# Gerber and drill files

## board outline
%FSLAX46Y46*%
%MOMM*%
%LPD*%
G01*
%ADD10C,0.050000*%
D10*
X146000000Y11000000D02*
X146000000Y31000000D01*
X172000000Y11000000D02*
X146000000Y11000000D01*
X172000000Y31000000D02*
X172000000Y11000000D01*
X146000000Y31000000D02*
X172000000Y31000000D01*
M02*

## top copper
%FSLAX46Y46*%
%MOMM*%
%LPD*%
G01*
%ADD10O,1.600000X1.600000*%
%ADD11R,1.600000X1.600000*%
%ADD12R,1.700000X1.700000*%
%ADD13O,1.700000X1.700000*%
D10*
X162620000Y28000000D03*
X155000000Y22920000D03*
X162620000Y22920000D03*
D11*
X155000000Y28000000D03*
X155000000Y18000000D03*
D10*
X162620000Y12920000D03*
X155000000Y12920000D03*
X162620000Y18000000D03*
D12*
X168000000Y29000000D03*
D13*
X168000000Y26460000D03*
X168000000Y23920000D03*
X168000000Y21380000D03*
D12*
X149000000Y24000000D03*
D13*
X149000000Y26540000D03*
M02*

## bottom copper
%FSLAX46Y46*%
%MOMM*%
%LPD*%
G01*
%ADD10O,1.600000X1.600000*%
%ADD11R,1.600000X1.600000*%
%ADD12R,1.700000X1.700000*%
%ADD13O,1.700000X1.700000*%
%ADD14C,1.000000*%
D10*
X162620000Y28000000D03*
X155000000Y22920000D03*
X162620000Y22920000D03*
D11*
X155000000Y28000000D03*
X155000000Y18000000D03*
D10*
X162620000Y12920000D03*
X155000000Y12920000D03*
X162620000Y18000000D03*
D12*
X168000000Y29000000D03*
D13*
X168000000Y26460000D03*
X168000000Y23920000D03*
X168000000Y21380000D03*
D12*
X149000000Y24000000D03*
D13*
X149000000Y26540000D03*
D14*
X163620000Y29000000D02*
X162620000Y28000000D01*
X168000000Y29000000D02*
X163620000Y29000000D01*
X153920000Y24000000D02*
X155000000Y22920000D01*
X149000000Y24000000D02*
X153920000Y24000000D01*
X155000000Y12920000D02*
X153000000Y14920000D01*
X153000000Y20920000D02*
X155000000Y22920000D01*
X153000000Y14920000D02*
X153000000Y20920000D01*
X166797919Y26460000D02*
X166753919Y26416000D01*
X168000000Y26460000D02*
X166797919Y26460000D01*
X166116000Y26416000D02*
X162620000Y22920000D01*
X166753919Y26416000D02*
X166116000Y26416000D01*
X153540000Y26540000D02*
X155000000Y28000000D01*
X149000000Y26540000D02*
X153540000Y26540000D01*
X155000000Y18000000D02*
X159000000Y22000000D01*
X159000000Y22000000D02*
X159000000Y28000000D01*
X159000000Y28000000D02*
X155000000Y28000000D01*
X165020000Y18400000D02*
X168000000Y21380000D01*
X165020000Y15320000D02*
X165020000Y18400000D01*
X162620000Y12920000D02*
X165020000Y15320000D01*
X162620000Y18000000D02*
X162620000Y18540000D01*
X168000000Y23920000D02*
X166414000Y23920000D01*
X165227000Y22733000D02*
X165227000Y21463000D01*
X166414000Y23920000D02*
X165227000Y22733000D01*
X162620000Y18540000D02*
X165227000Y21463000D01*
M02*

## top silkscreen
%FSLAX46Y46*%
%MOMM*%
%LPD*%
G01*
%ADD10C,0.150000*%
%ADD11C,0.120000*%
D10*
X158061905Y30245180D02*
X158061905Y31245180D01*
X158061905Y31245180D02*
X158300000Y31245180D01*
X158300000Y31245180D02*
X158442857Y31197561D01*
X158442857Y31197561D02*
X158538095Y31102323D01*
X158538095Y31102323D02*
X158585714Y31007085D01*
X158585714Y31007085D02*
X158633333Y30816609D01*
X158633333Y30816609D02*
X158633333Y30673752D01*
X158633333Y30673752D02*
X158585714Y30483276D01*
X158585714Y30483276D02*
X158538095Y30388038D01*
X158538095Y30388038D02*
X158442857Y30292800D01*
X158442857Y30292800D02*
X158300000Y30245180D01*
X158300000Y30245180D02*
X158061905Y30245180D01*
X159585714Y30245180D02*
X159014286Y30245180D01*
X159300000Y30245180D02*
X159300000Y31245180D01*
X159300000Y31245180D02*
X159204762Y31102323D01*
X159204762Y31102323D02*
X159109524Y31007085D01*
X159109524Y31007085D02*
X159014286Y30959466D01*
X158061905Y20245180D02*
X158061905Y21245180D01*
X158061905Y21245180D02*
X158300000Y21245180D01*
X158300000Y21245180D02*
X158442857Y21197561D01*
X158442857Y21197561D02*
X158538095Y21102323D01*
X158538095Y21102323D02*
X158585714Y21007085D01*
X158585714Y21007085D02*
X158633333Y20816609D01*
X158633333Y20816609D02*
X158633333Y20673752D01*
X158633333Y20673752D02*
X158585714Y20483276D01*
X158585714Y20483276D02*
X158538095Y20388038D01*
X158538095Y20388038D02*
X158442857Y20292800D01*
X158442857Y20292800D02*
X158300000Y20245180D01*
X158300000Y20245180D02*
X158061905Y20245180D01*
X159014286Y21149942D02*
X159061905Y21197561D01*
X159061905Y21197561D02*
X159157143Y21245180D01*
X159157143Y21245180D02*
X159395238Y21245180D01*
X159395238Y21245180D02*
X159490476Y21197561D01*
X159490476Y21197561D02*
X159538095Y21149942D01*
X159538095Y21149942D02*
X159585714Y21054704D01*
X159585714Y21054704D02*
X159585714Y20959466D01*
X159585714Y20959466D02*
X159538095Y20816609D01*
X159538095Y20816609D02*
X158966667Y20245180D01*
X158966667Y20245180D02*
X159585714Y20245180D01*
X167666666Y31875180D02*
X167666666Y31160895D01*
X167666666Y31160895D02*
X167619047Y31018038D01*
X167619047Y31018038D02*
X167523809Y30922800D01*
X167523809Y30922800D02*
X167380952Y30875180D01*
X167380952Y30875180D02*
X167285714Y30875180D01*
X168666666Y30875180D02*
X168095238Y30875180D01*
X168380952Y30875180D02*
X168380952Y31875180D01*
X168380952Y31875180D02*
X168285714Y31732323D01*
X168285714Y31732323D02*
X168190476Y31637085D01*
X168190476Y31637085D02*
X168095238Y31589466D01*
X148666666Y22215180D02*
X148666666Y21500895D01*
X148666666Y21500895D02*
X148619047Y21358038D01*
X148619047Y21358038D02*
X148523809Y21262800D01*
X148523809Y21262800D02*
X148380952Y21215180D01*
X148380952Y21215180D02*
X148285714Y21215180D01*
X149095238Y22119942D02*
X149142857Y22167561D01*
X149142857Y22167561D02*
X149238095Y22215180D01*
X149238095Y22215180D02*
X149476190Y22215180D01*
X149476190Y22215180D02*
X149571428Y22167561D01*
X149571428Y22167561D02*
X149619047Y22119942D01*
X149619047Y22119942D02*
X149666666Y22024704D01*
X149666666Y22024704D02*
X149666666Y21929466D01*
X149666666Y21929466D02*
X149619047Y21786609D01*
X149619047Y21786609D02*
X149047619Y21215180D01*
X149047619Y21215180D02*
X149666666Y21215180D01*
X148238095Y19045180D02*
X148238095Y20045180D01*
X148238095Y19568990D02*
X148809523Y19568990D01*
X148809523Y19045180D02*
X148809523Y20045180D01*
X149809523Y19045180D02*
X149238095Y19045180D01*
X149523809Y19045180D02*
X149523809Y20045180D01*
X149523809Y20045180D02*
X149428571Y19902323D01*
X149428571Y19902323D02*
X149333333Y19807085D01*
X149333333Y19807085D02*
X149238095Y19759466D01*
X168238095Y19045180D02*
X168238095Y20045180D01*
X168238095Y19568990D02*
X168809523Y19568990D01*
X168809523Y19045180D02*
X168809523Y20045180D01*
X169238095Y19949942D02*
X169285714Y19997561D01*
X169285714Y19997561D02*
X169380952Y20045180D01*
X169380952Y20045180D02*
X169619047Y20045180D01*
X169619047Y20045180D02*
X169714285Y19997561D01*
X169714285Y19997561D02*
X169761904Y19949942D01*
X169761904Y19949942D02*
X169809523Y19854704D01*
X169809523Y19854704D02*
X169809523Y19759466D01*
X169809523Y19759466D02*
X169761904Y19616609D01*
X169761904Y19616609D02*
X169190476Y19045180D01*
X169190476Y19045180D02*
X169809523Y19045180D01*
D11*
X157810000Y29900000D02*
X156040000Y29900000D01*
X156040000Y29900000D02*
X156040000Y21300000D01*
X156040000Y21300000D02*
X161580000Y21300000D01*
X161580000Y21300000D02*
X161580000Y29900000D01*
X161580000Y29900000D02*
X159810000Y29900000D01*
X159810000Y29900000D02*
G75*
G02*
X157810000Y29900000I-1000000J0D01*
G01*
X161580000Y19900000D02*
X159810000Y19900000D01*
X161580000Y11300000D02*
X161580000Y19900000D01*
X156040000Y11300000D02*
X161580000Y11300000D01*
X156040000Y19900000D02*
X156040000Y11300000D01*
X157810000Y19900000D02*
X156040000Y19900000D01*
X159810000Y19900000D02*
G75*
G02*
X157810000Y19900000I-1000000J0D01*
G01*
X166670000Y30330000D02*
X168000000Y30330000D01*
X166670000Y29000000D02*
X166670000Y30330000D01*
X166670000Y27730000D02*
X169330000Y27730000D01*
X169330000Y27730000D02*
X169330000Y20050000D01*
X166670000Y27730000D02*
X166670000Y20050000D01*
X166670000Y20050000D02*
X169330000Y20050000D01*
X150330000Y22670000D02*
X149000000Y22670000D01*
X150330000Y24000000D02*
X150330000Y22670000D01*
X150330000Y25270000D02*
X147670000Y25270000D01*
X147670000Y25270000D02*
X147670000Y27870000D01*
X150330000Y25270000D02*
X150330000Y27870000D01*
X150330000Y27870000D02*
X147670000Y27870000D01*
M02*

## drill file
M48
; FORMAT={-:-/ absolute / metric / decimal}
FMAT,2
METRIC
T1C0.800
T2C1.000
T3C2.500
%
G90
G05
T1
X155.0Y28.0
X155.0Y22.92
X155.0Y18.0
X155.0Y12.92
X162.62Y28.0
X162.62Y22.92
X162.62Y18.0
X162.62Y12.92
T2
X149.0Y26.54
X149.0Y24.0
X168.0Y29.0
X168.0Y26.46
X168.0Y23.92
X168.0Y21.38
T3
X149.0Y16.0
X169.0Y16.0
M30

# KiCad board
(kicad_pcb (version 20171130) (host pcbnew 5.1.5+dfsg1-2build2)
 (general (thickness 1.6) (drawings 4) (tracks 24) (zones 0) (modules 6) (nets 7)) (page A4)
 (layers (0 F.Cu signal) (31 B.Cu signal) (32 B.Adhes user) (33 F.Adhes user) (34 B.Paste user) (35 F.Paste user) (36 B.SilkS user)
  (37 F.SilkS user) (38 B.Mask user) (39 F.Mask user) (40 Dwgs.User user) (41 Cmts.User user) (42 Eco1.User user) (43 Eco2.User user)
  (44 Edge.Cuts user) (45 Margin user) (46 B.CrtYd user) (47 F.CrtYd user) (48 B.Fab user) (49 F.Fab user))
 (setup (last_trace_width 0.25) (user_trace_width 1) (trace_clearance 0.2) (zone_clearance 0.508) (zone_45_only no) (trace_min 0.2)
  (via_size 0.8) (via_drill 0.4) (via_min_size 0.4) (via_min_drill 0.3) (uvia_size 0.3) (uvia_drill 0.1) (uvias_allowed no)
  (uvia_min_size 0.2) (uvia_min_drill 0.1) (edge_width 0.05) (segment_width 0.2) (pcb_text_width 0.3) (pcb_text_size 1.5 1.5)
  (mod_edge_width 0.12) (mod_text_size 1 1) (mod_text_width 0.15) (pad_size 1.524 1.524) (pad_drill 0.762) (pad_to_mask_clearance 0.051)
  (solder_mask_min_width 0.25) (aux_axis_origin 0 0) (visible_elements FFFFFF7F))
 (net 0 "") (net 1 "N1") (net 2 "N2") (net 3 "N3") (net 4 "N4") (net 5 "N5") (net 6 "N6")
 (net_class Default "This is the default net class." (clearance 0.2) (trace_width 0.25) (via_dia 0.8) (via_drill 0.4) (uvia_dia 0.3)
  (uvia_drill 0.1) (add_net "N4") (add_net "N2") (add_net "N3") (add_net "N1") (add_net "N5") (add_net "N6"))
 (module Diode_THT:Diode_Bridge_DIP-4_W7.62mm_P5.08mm (layer F.Cu) (at 155 -28)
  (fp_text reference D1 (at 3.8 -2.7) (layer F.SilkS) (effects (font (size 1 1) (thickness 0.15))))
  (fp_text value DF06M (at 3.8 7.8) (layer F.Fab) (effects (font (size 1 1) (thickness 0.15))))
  (fp_line (start 2.81 -1.9) (end 1.04 -1.9) (layer F.SilkS) (width 0.12))
  (fp_line (start 1.04 -1.9) (end 1.04 6.7) (layer F.SilkS) (width 0.12))
  (fp_line (start 1.04 6.7) (end 6.58 6.7) (layer F.SilkS) (width 0.12))
  (fp_line (start 6.58 6.7) (end 6.58 -1.9) (layer F.SilkS) (width 0.12))
  (fp_line (start 6.58 -1.9) (end 4.81 -1.9) (layer F.SilkS) (width 0.12))
  (fp_arc (start 3.81 -1.9) (end 2.81 -1.9) (angle -180) (layer F.SilkS) (width 0.12))
  (pad 4 thru_hole oval (at 7.62 0) (size 1.6 1.6) (drill 0.8) (layers *.Cu *.Mask) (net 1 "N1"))
  (pad 2 thru_hole oval (at 0 5.08) (size 1.6 1.6) (drill 0.8) (layers *.Cu *.Mask) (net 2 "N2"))
  (pad 3 thru_hole oval (at 7.62 5.08) (size 1.6 1.6) (drill 0.8) (layers *.Cu *.Mask) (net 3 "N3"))
  (pad 1 thru_hole rect (at 0 0) (size 1.6 1.6) (drill 0.8) (layers *.Cu *.Mask) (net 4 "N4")))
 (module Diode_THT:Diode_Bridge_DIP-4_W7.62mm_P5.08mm (layer F.Cu) (at 155 -18)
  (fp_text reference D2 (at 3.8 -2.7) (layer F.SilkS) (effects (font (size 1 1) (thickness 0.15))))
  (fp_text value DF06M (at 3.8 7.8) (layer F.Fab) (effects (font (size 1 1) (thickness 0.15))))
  (fp_line (start 6.58 -1.9) (end 4.81 -1.9) (layer F.SilkS) (width 0.12))
  (fp_line (start 6.58 6.7) (end 6.58 -1.9) (layer F.SilkS) (width 0.12))
  (fp_line (start 1.04 6.7) (end 6.58 6.7) (layer F.SilkS) (width 0.12))
  (fp_line (start 1.04 -1.9) (end 1.04 6.7) (layer F.SilkS) (width 0.12))
  (fp_line (start 2.81 -1.9) (end 1.04 -1.9) (layer F.SilkS) (width 0.12))
  (fp_arc (start 3.81 -1.9) (end 2.81 -1.9) (angle -180) (layer F.SilkS) (width 0.12))
  (pad 1 thru_hole rect (at 0 0) (size 1.6 1.6) (drill 0.8) (layers *.Cu *.Mask) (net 4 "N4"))
  (pad 3 thru_hole oval (at 7.62 5.08) (size 1.6 1.6) (drill 0.8) (layers *.Cu *.Mask) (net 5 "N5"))
  (pad 2 thru_hole oval (at 0 5.08) (size 1.6 1.6) (drill 0.8) (layers *.Cu *.Mask) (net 2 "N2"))
  (pad 4 thru_hole oval (at 7.62 0) (size 1.6 1.6) (drill 0.8) (layers *.Cu *.Mask) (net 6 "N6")))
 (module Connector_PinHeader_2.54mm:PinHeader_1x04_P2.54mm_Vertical (layer F.Cu) (at 168 -29)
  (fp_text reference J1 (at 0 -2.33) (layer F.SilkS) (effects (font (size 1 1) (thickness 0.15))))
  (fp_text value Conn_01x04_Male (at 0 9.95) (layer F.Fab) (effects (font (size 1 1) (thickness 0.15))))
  (fp_line (start -1.33 -1.33) (end 0 -1.33) (layer F.SilkS) (width 0.12))
  (fp_line (start -1.33 0) (end -1.33 -1.33) (layer F.SilkS) (width 0.12))
  (fp_line (start -1.33 1.27) (end 1.33 1.27) (layer F.SilkS) (width 0.12))
  (fp_line (start 1.33 1.27) (end 1.33 8.95) (layer F.SilkS) (width 0.12))
  (fp_line (start -1.33 1.27) (end -1.33 8.95) (layer F.SilkS) (width 0.12))
  (fp_line (start -1.33 8.95) (end 1.33 8.95) (layer F.SilkS) (width 0.12))
  (pad 1 thru_hole rect (at 0 0) (size 1.7 1.7) (drill 1) (layers *.Cu *.Mask) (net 1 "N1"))
  (pad 2 thru_hole oval (at 0 2.54) (size 1.7 1.7) (drill 1) (layers *.Cu *.Mask) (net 3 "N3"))
  (pad 3 thru_hole oval (at 0 5.08) (size 1.7 1.7) (drill 1) (layers *.Cu *.Mask) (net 6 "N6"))
  (pad 4 thru_hole oval (at 0 7.62) (size 1.7 1.7) (drill 1) (layers *.Cu *.Mask) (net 5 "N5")))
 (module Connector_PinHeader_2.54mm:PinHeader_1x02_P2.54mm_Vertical (layer F.Cu) (at 149 -24 180)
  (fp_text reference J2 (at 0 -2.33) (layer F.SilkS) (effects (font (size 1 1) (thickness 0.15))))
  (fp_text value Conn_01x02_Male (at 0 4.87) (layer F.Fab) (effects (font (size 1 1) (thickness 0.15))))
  (fp_line (start -1.33 -1.33) (end 0 -1.33) (layer F.SilkS) (width 0.12))
  (fp_line (start -1.33 0) (end -1.33 -1.33) (layer F.SilkS) (width 0.12))
  (fp_line (start -1.33 1.27) (end 1.33 1.27) (layer F.SilkS) (width 0.12))
  (fp_line (start 1.33 1.27) (end 1.33 3.87) (layer F.SilkS) (width 0.12))
  (fp_line (start -1.33 1.27) (end -1.33 3.87) (layer F.SilkS) (width 0.12))
  (fp_line (start -1.33 3.87) (end 1.33 3.87) (layer F.SilkS) (width 0.12))
  (pad 1 thru_hole rect (at 0 0 180) (size 1.7 1.7) (drill 1) (layers *.Cu *.Mask) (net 2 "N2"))
  (pad 2 thru_hole oval (at 0 2.54 180) (size 1.7 1.7) (drill 1) (layers *.Cu *.Mask) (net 4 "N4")))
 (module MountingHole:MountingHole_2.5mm (layer F.Cu) (at 149 -16)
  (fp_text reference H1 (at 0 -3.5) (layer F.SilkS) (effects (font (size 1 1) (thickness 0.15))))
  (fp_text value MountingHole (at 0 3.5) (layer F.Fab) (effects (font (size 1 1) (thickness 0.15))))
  (pad 1 np_thru_hole circle (at 0 0) (size 2.5 2.5) (drill 2.5) (layers *.Cu *.Mask)))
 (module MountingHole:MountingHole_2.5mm (layer F.Cu) (at 169 -16)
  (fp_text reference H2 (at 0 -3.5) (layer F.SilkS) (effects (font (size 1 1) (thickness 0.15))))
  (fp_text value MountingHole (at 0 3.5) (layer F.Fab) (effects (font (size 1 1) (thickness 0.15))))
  (pad 1 np_thru_hole circle (at 0 0) (size 2.5 2.5) (drill 2.5) (layers *.Cu *.Mask)))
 (gr_line (start 146 -11) (end 146 -31) (layer Edge.Cuts) (width 0.05))
 (gr_line (start 172 -11) (end 146 -11) (layer Edge.Cuts) (width 0.05))
 (gr_line (start 172 -31) (end 172 -11) (layer Edge.Cuts) (width 0.05))
 (gr_line (start 146 -31) (end 172 -31) (layer Edge.Cuts) (width 0.05))
 (segment (start 163.62 -29) (end 162.62 -28) (width 1) (layer B.Cu) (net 1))
 (segment (start 168 -29) (end 163.62 -29) (width 1) (layer B.Cu) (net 1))
 (segment (start 153.92 -24) (end 155 -22.92) (width 1) (layer B.Cu) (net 2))
 (segment (start 149 -24) (end 153.92 -24) (width 1) (layer B.Cu) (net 2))
 (segment (start 155 -12.92) (end 153 -14.92) (width 1) (layer B.Cu) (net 2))
 (segment (start 153 -20.92) (end 155 -22.92) (width 1) (layer B.Cu) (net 2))
 (segment (start 153 -14.92) (end 153 -20.92) (width 1) (layer B.Cu) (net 2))
 (segment (start 166.797919 -26.46) (end 166.753919 -26.416) (width 1) (layer B.Cu) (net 3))
 (segment (start 168 -26.46) (end 166.797919 -26.46) (width 1) (layer B.Cu) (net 3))
 (segment (start 166.116 -26.416) (end 162.62 -22.92) (width 1) (layer B.Cu) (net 3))
 (segment (start 166.753919 -26.416) (end 166.116 -26.416) (width 1) (layer B.Cu) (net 3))
 (segment (start 153.54 -26.54) (end 155 -28) (width 1) (layer B.Cu) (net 4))
 (segment (start 149 -26.54) (end 153.54 -26.54) (width 1) (layer B.Cu) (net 4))
 (segment (start 155 -18) (end 159 -22) (width 1) (layer B.Cu) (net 4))
 (segment (start 159 -22) (end 159 -28) (width 1) (layer B.Cu) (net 4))
 (segment (start 159 -28) (end 155 -28) (width 1) (layer B.Cu) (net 4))
 (segment (start 165.02 -18.4) (end 168 -21.38) (width 1) (layer B.Cu) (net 5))
 (segment (start 165.02 -15.32) (end 165.02 -18.4) (width 1) (layer B.Cu) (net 5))
 (segment (start 162.62 -12.92) (end 165.02 -15.32) (width 1) (layer B.Cu) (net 5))
 (segment (start 162.62 -18) (end 162.62 -18.54) (width 1) (layer B.Cu) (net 6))
 (segment (start 168 -23.92) (end 166.414 -23.92) (width 1) (layer B.Cu) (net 6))
 (segment (start 165.227 -22.733) (end 165.227 -21.463) (width 1) (layer B.Cu) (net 6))
 (segment (start 166.414 -23.92) (end 165.227 -22.733) (width 1) (layer B.Cu) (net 6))
 (segment (start 162.62 -18.54) (end 165.227 -21.463) (width 1) (layer B.Cu) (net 6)))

